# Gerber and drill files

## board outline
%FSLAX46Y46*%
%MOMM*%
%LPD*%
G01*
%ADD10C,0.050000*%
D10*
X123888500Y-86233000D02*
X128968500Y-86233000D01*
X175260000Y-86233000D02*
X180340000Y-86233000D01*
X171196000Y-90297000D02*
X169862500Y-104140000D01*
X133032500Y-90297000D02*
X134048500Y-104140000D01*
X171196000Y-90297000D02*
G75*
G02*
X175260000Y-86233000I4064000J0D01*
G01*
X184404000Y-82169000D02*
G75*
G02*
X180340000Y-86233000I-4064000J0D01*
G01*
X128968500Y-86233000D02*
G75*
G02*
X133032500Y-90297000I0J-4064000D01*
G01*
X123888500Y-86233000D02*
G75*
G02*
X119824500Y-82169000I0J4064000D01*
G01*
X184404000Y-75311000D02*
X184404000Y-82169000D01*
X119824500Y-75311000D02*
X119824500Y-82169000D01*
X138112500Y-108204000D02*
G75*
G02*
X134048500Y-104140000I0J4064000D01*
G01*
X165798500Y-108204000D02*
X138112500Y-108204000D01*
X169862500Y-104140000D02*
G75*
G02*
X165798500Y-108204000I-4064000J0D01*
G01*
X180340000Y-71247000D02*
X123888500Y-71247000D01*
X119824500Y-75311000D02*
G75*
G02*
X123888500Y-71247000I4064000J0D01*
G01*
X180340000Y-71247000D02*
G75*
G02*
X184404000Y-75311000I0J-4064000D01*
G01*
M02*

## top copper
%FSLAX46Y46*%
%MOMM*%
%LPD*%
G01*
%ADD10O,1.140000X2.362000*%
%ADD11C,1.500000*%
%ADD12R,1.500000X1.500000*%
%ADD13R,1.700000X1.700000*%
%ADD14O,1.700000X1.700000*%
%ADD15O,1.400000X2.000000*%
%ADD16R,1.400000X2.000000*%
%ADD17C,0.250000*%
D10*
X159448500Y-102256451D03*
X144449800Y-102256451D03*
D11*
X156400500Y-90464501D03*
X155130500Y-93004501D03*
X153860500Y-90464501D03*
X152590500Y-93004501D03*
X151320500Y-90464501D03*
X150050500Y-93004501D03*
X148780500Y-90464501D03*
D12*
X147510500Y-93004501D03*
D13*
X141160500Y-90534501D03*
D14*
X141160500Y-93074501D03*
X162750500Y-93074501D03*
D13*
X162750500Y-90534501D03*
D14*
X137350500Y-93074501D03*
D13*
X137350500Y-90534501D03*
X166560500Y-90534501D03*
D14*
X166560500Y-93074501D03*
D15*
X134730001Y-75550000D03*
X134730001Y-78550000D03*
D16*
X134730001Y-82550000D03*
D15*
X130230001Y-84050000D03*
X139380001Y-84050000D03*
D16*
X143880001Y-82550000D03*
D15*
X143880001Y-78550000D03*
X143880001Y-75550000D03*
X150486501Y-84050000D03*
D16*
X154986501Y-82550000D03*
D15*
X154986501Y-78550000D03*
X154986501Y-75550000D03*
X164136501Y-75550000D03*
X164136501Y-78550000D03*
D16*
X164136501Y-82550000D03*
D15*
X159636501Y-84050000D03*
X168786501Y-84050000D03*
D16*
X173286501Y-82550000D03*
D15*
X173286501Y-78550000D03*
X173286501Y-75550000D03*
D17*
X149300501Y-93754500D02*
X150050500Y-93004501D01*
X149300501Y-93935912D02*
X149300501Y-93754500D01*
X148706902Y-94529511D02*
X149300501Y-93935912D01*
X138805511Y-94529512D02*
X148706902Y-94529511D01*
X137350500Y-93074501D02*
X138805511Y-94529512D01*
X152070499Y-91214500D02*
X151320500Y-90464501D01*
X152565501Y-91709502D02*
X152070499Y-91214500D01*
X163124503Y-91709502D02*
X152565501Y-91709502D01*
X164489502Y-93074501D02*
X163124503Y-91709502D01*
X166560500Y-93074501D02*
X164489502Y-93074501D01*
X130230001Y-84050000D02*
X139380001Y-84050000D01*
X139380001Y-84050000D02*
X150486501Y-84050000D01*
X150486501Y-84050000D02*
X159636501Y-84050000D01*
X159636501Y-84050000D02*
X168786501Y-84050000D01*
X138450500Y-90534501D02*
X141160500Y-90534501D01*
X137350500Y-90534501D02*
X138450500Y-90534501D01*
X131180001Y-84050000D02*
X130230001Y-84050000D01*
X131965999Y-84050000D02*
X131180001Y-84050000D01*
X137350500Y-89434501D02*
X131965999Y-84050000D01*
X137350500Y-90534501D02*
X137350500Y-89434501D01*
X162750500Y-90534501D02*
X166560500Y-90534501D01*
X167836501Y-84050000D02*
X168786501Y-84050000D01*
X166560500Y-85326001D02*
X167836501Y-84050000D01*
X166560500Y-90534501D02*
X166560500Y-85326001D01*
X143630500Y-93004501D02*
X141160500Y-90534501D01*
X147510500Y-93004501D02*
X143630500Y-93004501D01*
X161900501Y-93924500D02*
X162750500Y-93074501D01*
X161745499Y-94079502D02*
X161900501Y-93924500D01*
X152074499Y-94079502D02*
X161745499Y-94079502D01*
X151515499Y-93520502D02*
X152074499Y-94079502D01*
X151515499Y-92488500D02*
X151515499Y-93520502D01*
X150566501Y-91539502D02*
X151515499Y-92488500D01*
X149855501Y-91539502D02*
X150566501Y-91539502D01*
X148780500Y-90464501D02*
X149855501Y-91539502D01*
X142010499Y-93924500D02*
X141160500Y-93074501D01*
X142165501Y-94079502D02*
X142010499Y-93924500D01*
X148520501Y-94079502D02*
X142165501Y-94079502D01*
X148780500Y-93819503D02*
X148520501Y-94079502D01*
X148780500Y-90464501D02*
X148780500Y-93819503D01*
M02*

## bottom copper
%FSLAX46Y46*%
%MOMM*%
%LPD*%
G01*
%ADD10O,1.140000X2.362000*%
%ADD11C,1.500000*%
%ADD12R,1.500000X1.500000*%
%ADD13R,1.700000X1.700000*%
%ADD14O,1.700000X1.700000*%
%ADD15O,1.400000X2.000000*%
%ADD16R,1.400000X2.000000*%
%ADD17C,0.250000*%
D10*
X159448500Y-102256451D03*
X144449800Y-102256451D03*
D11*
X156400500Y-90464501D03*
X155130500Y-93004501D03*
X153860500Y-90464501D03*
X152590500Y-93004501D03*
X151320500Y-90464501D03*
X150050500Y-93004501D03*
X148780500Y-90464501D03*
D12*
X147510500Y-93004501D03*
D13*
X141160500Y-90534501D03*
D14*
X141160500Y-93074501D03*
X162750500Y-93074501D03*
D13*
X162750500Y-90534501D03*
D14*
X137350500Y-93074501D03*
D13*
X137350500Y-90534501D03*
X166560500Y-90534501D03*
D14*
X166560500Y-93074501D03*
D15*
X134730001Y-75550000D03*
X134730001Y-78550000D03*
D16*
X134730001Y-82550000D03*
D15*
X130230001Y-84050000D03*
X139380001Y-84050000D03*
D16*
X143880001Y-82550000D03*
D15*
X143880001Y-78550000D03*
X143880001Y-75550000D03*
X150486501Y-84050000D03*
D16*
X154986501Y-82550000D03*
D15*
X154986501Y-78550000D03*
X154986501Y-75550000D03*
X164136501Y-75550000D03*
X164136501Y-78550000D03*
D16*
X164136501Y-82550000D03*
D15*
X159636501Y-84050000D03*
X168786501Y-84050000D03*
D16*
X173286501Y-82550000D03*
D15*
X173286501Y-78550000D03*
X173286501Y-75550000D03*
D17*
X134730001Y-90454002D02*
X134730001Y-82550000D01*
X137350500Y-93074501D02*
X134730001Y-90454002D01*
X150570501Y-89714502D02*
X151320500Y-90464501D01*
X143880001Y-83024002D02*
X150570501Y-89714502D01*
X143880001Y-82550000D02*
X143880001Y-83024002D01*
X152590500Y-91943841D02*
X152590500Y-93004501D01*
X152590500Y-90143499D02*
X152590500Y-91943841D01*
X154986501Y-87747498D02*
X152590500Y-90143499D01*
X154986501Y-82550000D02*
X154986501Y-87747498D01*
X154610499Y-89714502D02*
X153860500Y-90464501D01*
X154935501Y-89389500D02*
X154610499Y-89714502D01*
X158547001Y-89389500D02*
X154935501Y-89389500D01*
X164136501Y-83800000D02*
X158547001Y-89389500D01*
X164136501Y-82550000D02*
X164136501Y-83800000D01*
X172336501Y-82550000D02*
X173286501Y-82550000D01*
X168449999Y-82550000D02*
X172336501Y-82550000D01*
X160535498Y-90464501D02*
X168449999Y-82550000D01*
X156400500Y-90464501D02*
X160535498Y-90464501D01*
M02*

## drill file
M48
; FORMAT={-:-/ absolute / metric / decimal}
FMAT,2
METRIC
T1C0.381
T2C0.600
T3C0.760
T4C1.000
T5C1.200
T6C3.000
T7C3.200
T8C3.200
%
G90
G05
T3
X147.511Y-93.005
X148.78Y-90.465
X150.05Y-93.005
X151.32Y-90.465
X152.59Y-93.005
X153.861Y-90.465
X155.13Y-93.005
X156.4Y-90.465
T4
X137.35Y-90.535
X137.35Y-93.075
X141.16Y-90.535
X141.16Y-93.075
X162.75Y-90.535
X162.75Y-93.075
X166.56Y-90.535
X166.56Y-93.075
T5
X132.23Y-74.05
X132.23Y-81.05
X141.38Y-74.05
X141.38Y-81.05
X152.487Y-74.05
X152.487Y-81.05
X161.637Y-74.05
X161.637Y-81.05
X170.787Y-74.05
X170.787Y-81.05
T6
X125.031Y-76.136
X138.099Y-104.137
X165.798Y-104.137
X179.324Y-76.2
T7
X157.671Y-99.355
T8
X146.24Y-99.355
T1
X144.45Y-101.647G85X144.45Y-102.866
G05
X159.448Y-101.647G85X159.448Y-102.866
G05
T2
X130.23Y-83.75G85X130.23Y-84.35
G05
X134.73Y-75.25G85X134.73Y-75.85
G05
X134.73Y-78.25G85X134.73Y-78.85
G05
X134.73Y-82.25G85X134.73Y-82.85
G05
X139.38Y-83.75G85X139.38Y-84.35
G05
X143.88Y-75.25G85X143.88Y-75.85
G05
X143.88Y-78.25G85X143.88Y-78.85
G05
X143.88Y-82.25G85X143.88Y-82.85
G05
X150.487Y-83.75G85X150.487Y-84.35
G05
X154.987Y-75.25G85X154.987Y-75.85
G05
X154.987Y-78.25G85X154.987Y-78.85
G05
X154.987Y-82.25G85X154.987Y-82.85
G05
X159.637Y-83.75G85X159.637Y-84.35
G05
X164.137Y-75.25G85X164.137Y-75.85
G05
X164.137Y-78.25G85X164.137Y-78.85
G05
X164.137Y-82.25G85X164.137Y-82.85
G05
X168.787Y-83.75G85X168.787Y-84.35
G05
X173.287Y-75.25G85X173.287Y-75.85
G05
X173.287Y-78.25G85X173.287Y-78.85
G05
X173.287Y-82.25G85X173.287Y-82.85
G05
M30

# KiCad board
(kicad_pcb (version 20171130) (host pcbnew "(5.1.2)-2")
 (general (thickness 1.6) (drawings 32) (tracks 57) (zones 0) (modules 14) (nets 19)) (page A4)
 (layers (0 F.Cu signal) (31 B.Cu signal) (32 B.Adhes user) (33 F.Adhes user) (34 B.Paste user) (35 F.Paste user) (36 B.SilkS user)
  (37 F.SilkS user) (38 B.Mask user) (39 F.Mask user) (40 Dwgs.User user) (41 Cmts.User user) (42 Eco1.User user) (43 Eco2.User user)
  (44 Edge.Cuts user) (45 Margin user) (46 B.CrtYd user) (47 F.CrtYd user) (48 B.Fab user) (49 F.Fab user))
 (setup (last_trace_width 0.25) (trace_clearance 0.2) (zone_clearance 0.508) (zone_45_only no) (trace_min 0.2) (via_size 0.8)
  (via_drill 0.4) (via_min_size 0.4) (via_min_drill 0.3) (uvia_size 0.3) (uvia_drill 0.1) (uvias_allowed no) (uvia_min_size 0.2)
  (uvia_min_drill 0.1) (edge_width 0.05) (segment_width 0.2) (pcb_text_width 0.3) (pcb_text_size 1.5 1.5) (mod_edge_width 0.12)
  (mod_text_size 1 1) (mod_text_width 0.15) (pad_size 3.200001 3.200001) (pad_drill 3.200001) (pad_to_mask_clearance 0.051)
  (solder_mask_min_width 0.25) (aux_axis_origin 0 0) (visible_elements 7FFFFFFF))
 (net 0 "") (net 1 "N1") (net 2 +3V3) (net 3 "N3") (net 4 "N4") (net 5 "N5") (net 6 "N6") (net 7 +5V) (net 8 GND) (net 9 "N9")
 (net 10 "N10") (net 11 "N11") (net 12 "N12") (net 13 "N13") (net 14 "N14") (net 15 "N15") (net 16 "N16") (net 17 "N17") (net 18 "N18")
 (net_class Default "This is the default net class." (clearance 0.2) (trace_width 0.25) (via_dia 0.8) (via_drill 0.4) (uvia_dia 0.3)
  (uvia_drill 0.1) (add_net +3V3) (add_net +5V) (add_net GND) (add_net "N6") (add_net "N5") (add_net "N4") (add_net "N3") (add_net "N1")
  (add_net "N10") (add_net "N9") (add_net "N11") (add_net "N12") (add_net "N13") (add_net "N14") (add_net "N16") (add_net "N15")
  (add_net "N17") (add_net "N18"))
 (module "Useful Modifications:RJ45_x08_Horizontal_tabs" (layer F.Cu) (at 147.5105 93.004501)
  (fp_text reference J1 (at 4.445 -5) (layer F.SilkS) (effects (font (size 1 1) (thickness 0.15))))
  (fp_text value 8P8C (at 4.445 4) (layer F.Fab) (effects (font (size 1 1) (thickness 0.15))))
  (pad 10 thru_hole oval (at 11.938 9.25195) (size 1.14 2.362) (drill oval 0.381 1.6) (layers *.Cu *.Mask))
  (pad 9 thru_hole oval (at -3.0607 9.25195) (size 1.14 2.362) (drill oval 0.381 1.6) (layers *.Cu *.Mask))
  (pad 8 thru_hole circle (at 8.89 -2.54) (size 1.5 1.5) (drill 0.76) (layers *.Cu *.Mask) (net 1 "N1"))
  (pad 7 thru_hole circle (at 7.62 0) (size 1.5 1.5) (drill 0.76) (layers *.Cu *.Mask) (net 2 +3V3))
  (pad 6 thru_hole circle (at 6.35 -2.54) (size 1.5 1.5) (drill 0.76) (layers *.Cu *.Mask) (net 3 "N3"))
  (pad 5 thru_hole circle (at 5.08 0) (size 1.5 1.5) (drill 0.76) (layers *.Cu *.Mask) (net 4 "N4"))
  (pad 4 thru_hole circle (at 3.81 -2.54) (size 1.5 1.5) (drill 0.76) (layers *.Cu *.Mask) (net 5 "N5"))
  (pad 3 thru_hole circle (at 2.54 0) (size 1.5 1.5) (drill 0.76) (layers *.Cu *.Mask) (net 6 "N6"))
  (pad 2 thru_hole circle (at 1.27 -2.54) (size 1.5 1.5) (drill 0.76) (layers *.Cu *.Mask) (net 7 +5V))
  (pad 1 thru_hole rect (at 0 0) (size 1.5 1.5) (drill 0.76) (layers *.Cu *.Mask) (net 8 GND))
  (pad "" np_thru_hole circle (at -1.27 6.35) (size 3.200001 3.200001) (drill 3.200001) (layers *.Cu *.Mask))
  (pad "" np_thru_hole circle (at 10.16 6.35) (size 3.2 3.2) (drill 3.2) (layers *.Cu *.Mask)))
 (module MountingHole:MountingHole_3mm (layer F.Cu) (at 138.0985 104.1375)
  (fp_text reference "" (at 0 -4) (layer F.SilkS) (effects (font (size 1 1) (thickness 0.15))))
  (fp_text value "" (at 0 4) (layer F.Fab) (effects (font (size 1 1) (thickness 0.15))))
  (pad 1 np_thru_hole circle (at 0 0) (size 3 3) (drill 3) (layers *.Cu *.Mask)))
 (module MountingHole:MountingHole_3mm (layer F.Cu) (at 125.0315 76.1365)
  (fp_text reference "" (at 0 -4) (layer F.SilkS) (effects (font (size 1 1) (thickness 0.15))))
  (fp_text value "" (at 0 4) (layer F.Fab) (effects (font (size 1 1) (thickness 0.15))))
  (pad 1 np_thru_hole circle (at 0 0) (size 3 3) (drill 3) (layers *.Cu *.Mask)))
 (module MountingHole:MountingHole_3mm (layer F.Cu) (at 165.7985 104.1375)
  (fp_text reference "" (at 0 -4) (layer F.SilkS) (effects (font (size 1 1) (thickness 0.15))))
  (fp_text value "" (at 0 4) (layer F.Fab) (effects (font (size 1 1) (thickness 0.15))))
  (pad 1 np_thru_hole circle (at 0 0) (size 3 3) (drill 3) (layers *.Cu *.Mask)))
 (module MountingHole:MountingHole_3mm (layer F.Cu) (at 179.324 76.2)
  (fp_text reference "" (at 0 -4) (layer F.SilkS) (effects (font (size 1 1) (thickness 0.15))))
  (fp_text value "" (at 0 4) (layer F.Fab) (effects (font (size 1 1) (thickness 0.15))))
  (pad 1 np_thru_hole circle (at 0 0) (size 3 3) (drill 3) (layers *.Cu *.Mask)))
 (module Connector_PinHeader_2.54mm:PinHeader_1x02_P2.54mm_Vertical (layer F.Cu) (at 141.1605 90.534501)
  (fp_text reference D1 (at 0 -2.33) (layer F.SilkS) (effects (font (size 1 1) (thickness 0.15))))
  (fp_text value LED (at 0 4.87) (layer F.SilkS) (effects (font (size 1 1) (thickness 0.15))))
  (pad 1 thru_hole rect (at 0 0) (size 1.7 1.7) (drill 1) (layers *.Cu *.Mask) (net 8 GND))
  (pad 2 thru_hole oval (at 0 2.54) (size 1.7 1.7) (drill 1) (layers *.Cu *.Mask) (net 7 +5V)))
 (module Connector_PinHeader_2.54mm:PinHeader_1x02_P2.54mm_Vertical (layer F.Cu) (at 162.7505 90.534501)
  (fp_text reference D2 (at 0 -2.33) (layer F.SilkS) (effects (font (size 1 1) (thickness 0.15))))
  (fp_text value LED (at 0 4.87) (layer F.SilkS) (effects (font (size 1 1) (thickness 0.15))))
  (pad 2 thru_hole oval (at 0 2.54) (size 1.7 1.7) (drill 1) (layers *.Cu *.Mask) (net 7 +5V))
  (pad 1 thru_hole rect (at 0 0) (size 1.7 1.7) (drill 1) (layers *.Cu *.Mask) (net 8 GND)))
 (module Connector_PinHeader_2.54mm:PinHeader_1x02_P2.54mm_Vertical (layer F.Cu) (at 137.3505 90.534501)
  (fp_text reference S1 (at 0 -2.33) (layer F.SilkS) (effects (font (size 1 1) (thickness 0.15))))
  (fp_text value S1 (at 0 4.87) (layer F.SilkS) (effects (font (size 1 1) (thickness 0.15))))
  (pad 2 thru_hole oval (at 0 2.54) (size 1.7 1.7) (drill 1) (layers *.Cu *.Mask) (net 6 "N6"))
  (pad 1 thru_hole rect (at 0 0) (size 1.7 1.7) (drill 1) (layers *.Cu *.Mask) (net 8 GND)))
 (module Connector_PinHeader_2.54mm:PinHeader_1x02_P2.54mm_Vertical (layer F.Cu) (at 166.5605 90.534501)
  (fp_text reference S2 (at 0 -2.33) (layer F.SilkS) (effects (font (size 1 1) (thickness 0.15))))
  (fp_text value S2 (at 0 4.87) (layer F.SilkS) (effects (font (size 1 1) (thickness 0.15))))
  (pad 1 thru_hole rect (at 0 0) (size 1.7 1.7) (drill 1) (layers *.Cu *.Mask) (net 8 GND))
  (pad 2 thru_hole oval (at 0 2.54) (size 1.7 1.7) (drill 1) (layers *.Cu *.Mask) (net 5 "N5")))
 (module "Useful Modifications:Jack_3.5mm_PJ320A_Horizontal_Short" (layer F.Cu) (at 130.230001 82.55)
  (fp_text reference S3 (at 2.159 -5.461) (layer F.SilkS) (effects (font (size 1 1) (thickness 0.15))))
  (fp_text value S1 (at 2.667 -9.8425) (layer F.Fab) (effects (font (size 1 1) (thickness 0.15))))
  (pad "" np_thru_hole circle (at 2 -1.5 270) (size 1.2 1.2) (drill 1.2) (layers *.Cu *.Mask))
  (pad "" np_thru_hole circle (at 2 -8.5 270) (size 1.2 1.2) (drill 1.2) (layers *.Cu *.Mask))
  (pad R2 thru_hole oval (at 4.5 -7 270) (size 2 1.4) (drill oval 1.2 0.6) (layers *.Cu *.Mask) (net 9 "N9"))
  (pad R1 thru_hole oval (at 4.5 -4 270) (size 2 1.4) (drill oval 1.2 0.6) (layers *.Cu *.Mask) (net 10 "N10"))
  (pad T thru_hole rect (at 4.5 0 270) (size 2 1.4) (drill oval 1.2 0.6) (layers *.Cu *.Mask) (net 6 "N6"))
  (pad S thru_hole oval (at 0 1.5 270) (size 2 1.4) (drill oval 1.2 0.6) (layers *.Cu *.Mask) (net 8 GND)))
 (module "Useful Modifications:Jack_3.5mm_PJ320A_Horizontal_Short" (layer F.Cu) (at 139.380001 82.55)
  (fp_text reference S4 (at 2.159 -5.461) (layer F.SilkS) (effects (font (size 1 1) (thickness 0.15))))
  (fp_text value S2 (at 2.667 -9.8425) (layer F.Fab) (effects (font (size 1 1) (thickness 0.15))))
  (pad S thru_hole oval (at 0 1.5 270) (size 2 1.4) (drill oval 1.2 0.6) (layers *.Cu *.Mask) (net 8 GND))
  (pad T thru_hole rect (at 4.5 0 270) (size 2 1.4) (drill oval 1.2 0.6) (layers *.Cu *.Mask) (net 5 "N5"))
  (pad R1 thru_hole oval (at 4.5 -4 270) (size 2 1.4) (drill oval 1.2 0.6) (layers *.Cu *.Mask) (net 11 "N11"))
  (pad R2 thru_hole oval (at 4.5 -7 270) (size 2 1.4) (drill oval 1.2 0.6) (layers *.Cu *.Mask) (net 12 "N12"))
  (pad "" np_thru_hole circle (at 2 -8.5 270) (size 1.2 1.2) (drill 1.2) (layers *.Cu *.Mask))
  (pad "" np_thru_hole circle (at 2 -1.5 270) (size 1.2 1.2) (drill 1.2) (layers *.Cu *.Mask)))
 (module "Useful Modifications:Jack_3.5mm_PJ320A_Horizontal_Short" (layer F.Cu) (at 150.486501 82.55)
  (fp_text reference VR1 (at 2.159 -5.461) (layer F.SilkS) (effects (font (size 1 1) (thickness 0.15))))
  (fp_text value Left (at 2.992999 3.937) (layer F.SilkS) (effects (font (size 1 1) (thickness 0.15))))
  (pad S thru_hole oval (at 0 1.5 270) (size 2 1.4) (drill oval 1.2 0.6) (layers *.Cu *.Mask) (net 8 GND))
  (pad T thru_hole rect (at 4.5 0 270) (size 2 1.4) (drill oval 1.2 0.6) (layers *.Cu *.Mask) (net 4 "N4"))
  (pad R1 thru_hole oval (at 4.5 -4 270) (size 2 1.4) (drill oval 1.2 0.6) (layers *.Cu *.Mask) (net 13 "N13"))
  (pad R2 thru_hole oval (at 4.5 -7 270) (size 2 1.4) (drill oval 1.2 0.6) (layers *.Cu *.Mask) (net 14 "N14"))
  (pad "" np_thru_hole circle (at 2 -8.5 270) (size 1.2 1.2) (drill 1.2) (layers *.Cu *.Mask))
  (pad "" np_thru_hole circle (at 2 -1.5 270) (size 1.2 1.2) (drill 1.2) (layers *.Cu *.Mask)))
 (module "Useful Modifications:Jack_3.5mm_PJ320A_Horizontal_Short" (layer F.Cu) (at 159.636501 82.55)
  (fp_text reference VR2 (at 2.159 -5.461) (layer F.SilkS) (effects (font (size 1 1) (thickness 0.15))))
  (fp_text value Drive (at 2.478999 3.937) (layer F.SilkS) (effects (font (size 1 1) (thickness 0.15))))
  (pad "" np_thru_hole circle (at 2 -1.5 270) (size 1.2 1.2) (drill 1.2) (layers *.Cu *.Mask))
  (pad "" np_thru_hole circle (at 2 -8.5 270) (size 1.2 1.2) (drill 1.2) (layers *.Cu *.Mask))
  (pad R2 thru_hole oval (at 4.5 -7 270) (size 2 1.4) (drill oval 1.2 0.6) (layers *.Cu *.Mask) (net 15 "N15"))
  (pad R1 thru_hole oval (at 4.5 -4 270) (size 2 1.4) (drill oval 1.2 0.6) (layers *.Cu *.Mask) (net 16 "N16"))
  (pad T thru_hole rect (at 4.5 0 270) (size 2 1.4) (drill oval 1.2 0.6) (layers *.Cu *.Mask) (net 3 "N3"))
  (pad S thru_hole oval (at 0 1.5 270) (size 2 1.4) (drill oval 1.2 0.6) (layers *.Cu *.Mask) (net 8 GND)))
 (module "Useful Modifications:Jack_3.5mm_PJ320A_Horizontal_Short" (layer F.Cu) (at 168.786501 82.55)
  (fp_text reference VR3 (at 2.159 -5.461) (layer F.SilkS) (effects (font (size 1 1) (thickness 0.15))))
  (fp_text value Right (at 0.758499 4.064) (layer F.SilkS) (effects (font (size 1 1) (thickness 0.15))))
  (pad S thru_hole oval (at 0 1.5 270) (size 2 1.4) (drill oval 1.2 0.6) (layers *.Cu *.Mask) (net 8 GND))
  (pad T thru_hole rect (at 4.5 0 270) (size 2 1.4) (drill oval 1.2 0.6) (layers *.Cu *.Mask) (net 1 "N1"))
  (pad R1 thru_hole oval (at 4.5 -4 270) (size 2 1.4) (drill oval 1.2 0.6) (layers *.Cu *.Mask) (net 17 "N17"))
  (pad R2 thru_hole oval (at 4.5 -7 270) (size 2 1.4) (drill oval 1.2 0.6) (layers *.Cu *.Mask) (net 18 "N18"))
  (pad "" np_thru_hole circle (at 2 -8.5 270) (size 1.2 1.2) (drill 1.2) (layers *.Cu *.Mask))
  (pad "" np_thru_hole circle (at 2 -1.5 270) (size 1.2 1.2) (drill 1.2) (layers *.Cu *.Mask)))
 (gr_line (start 123.8885 86.233) (end 128.9685 86.233) (layer Edge.Cuts) (width 0.05))
 (gr_line (start 175.26 86.233) (end 180.34 86.233) (layer Edge.Cuts) (width 0.05))
 (gr_line (start 171.196 90.297) (end 169.8625 104.14) (layer Edge.Cuts) (width 0.05))
 (gr_line (start 133.0325 90.297) (end 134.0485 104.14) (layer Edge.Cuts) (width 0.05))
 (gr_arc (start 175.26 90.297) (end 175.26 86.233) (angle -90) (layer Edge.Cuts) (width 0.05))
 (gr_arc (start 180.34 82.169) (end 180.34 86.233) (angle -90) (layer Edge.Cuts) (width 0.05))
 (gr_arc (start 128.9685 90.297) (end 133.0325 90.297) (angle -90) (layer Edge.Cuts) (width 0.05))
 (gr_arc (start 123.8885 82.169) (end 119.8245 82.169) (angle -90) (layer Edge.Cuts) (width 0.05))
 (gr_line (start 184.404 75.311) (end 184.404 82.169) (layer Edge.Cuts) (width 0.05))
 (gr_line (start 119.8245 75.311) (end 119.8245 82.169) (layer Edge.Cuts) (width 0.05))
 (gr_arc (start 138.1125 104.14) (end 134.0485 104.14) (angle -90) (layer Edge.Cuts) (width 0.05))
 (gr_line (start 165.7985 108.204) (end 138.1125 108.204) (layer Edge.Cuts) (width 0.05))
 (gr_arc (start 165.7985 104.14) (end 165.7985 108.204) (angle -90) (layer Edge.Cuts) (width 0.05))
 (gr_line (start 180.34 71.247) (end 123.8885 71.247) (layer Edge.Cuts) (width 0.05))
 (gr_arc (start 123.8885 75.311) (end 123.8885 71.247) (angle -90) (layer Edge.Cuts) (width 0.05))
 (gr_arc (start 180.34 75.311) (end 184.404 75.311) (angle -90) (layer Edge.Cuts) (width 0.05))
 (segment (start 149.300501 93.7545) (end 150.0505 93.004501) (width 0.25) (layer F.Cu) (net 6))
 (segment (start 149.300501 93.935912) (end 149.300501 93.7545) (width 0.25) (layer F.Cu) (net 6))
 (segment (start 148.706902 94.529511) (end 149.300501 93.935912) (width 0.25) (layer F.Cu) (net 6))
 (segment (start 138.805511 94.529512) (end 148.706902 94.529511) (width 0.25) (layer F.Cu) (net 6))
 (segment (start 137.3505 93.074501) (end 138.805511 94.529512) (width 0.25) (layer F.Cu) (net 6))
 (segment (start 134.730001 90.454002) (end 134.730001 82.55) (width 0.25) (layer B.Cu) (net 6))
 (segment (start 137.3505 93.074501) (end 134.730001 90.454002) (width 0.25) (layer B.Cu) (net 6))
 (segment (start 152.070499 91.2145) (end 151.3205 90.464501) (width 0.25) (layer F.Cu) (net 5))
 (segment (start 152.565501 91.709502) (end 152.070499 91.2145) (width 0.25) (layer F.Cu) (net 5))
 (segment (start 163.124503 91.709502) (end 152.565501 91.709502) (width 0.25) (layer F.Cu) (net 5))
 (segment (start 164.489502 93.074501) (end 163.124503 91.709502) (width 0.25) (layer F.Cu) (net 5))
 (segment (start 166.5605 93.074501) (end 164.489502 93.074501) (width 0.25) (layer F.Cu) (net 5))
 (segment (start 150.570501 89.714502) (end 151.3205 90.464501) (width 0.25) (layer B.Cu) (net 5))
 (segment (start 143.880001 83.024002) (end 150.570501 89.714502) (width 0.25) (layer B.Cu) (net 5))
 (segment (start 143.880001 82.55) (end 143.880001 83.024002) (width 0.25) (layer B.Cu) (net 5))
 (segment (start 152.5905 91.943841) (end 152.5905 93.004501) (width 0.25) (layer B.Cu) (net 4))
 (segment (start 152.5905 90.143499) (end 152.5905 91.943841) (width 0.25) (layer B.Cu) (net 4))
 (segment (start 154.986501 87.747498) (end 152.5905 90.143499) (width 0.25) (layer B.Cu) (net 4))
 (segment (start 154.986501 82.55) (end 154.986501 87.747498) (width 0.25) (layer B.Cu) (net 4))
 (segment (start 154.610499 89.714502) (end 153.8605 90.464501) (width 0.25) (layer B.Cu) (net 3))
 (segment (start 154.935501 89.3895) (end 154.610499 89.714502) (width 0.25) (layer B.Cu) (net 3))
 (segment (start 158.547001 89.3895) (end 154.935501 89.3895) (width 0.25) (layer B.Cu) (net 3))
 (segment (start 164.136501 83.8) (end 158.547001 89.3895) (width 0.25) (layer B.Cu) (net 3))
 (segment (start 164.136501 82.55) (end 164.136501 83.8) (width 0.25) (layer B.Cu) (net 3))
 (segment (start 172.336501 82.55) (end 173.286501 82.55) (width 0.25) (layer B.Cu) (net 1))
 (segment (start 168.449999 82.55) (end 172.336501 82.55) (width 0.25) (layer B.Cu) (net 1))
 (segment (start 160.535498 90.464501) (end 168.449999 82.55) (width 0.25) (layer B.Cu) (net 1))
 (segment (start 156.4005 90.464501) (end 160.535498 90.464501) (width 0.25) (layer B.Cu) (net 1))
 (segment (start 130.230001 84.05) (end 139.380001 84.05) (width 0.25) (layer F.Cu) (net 8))
 (segment (start 139.380001 84.05) (end 150.486501 84.05) (width 0.25) (layer F.Cu) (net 8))
 (segment (start 150.486501 84.05) (end 159.636501 84.05) (width 0.25) (layer F.Cu) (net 8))
 (segment (start 159.636501 84.05) (end 168.786501 84.05) (width 0.25) (layer F.Cu) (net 8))
 (segment (start 138.4505 90.534501) (end 141.1605 90.534501) (width 0.25) (layer F.Cu) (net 8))
 (segment (start 137.3505 90.534501) (end 138.4505 90.534501) (width 0.25) (layer F.Cu) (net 8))
 (segment (start 131.180001 84.05) (end 130.230001 84.05) (width 0.25) (layer F.Cu) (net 8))
 (segment (start 131.965999 84.05) (end 131.180001 84.05) (width 0.25) (layer F.Cu) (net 8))
 (segment (start 137.3505 89.434501) (end 131.965999 84.05) (width 0.25) (layer F.Cu) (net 8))
 (segment (start 137.3505 90.534501) (end 137.3505 89.434501) (width 0.25) (layer F.Cu) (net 8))
 (segment (start 162.7505 90.534501) (end 166.5605 90.534501) (width 0.25) (layer F.Cu) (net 8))
 (segment (start 167.836501 84.05) (end 168.786501 84.05) (width 0.25) (layer F.Cu) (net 8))
 (segment (start 166.5605 85.326001) (end 167.836501 84.05) (width 0.25) (layer F.Cu) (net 8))
 (segment (start 166.5605 90.534501) (end 166.5605 85.326001) (width 0.25) (layer F.Cu) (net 8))
 (segment (start 143.6305 93.004501) (end 141.1605 90.534501) (width 0.25) (layer F.Cu) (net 8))
 (segment (start 147.5105 93.004501) (end 143.6305 93.004501) (width 0.25) (layer F.Cu) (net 8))
 (segment (start 161.900501 93.9245) (end 162.7505 93.074501) (width 0.25) (layer F.Cu) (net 7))
 (segment (start 161.745499 94.079502) (end 161.900501 93.9245) (width 0.25) (layer F.Cu) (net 7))
 (segment (start 152.074499 94.079502) (end 161.745499 94.079502) (width 0.25) (layer F.Cu) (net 7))
 (segment (start 151.515499 93.520502) (end 152.074499 94.079502) (width 0.25) (layer F.Cu) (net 7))
 (segment (start 151.515499 92.4885) (end 151.515499 93.520502) (width 0.25) (layer F.Cu) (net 7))
 (segment (start 150.566501 91.539502) (end 151.515499 92.4885) (width 0.25) (layer F.Cu) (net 7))
 (segment (start 149.855501 91.539502) (end 150.566501 91.539502) (width 0.25) (layer F.Cu) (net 7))
 (segment (start 148.7805 90.464501) (end 149.855501 91.539502) (width 0.25) (layer F.Cu) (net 7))
 (segment (start 142.010499 93.9245) (end 141.1605 93.074501) (width 0.25) (layer F.Cu) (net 7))
 (segment (start 142.165501 94.079502) (end 142.010499 93.9245) (width 0.25) (layer F.Cu) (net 7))
 (segment (start 148.520501 94.079502) (end 142.165501 94.079502) (width 0.25) (layer F.Cu) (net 7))
 (segment (start 148.7805 93.819503) (end 148.520501 94.079502) (width 0.25) (layer F.Cu) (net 7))
 (segment (start 148.7805 90.464501) (end 148.7805 93.819503) (width 0.25) (layer F.Cu) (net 7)))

